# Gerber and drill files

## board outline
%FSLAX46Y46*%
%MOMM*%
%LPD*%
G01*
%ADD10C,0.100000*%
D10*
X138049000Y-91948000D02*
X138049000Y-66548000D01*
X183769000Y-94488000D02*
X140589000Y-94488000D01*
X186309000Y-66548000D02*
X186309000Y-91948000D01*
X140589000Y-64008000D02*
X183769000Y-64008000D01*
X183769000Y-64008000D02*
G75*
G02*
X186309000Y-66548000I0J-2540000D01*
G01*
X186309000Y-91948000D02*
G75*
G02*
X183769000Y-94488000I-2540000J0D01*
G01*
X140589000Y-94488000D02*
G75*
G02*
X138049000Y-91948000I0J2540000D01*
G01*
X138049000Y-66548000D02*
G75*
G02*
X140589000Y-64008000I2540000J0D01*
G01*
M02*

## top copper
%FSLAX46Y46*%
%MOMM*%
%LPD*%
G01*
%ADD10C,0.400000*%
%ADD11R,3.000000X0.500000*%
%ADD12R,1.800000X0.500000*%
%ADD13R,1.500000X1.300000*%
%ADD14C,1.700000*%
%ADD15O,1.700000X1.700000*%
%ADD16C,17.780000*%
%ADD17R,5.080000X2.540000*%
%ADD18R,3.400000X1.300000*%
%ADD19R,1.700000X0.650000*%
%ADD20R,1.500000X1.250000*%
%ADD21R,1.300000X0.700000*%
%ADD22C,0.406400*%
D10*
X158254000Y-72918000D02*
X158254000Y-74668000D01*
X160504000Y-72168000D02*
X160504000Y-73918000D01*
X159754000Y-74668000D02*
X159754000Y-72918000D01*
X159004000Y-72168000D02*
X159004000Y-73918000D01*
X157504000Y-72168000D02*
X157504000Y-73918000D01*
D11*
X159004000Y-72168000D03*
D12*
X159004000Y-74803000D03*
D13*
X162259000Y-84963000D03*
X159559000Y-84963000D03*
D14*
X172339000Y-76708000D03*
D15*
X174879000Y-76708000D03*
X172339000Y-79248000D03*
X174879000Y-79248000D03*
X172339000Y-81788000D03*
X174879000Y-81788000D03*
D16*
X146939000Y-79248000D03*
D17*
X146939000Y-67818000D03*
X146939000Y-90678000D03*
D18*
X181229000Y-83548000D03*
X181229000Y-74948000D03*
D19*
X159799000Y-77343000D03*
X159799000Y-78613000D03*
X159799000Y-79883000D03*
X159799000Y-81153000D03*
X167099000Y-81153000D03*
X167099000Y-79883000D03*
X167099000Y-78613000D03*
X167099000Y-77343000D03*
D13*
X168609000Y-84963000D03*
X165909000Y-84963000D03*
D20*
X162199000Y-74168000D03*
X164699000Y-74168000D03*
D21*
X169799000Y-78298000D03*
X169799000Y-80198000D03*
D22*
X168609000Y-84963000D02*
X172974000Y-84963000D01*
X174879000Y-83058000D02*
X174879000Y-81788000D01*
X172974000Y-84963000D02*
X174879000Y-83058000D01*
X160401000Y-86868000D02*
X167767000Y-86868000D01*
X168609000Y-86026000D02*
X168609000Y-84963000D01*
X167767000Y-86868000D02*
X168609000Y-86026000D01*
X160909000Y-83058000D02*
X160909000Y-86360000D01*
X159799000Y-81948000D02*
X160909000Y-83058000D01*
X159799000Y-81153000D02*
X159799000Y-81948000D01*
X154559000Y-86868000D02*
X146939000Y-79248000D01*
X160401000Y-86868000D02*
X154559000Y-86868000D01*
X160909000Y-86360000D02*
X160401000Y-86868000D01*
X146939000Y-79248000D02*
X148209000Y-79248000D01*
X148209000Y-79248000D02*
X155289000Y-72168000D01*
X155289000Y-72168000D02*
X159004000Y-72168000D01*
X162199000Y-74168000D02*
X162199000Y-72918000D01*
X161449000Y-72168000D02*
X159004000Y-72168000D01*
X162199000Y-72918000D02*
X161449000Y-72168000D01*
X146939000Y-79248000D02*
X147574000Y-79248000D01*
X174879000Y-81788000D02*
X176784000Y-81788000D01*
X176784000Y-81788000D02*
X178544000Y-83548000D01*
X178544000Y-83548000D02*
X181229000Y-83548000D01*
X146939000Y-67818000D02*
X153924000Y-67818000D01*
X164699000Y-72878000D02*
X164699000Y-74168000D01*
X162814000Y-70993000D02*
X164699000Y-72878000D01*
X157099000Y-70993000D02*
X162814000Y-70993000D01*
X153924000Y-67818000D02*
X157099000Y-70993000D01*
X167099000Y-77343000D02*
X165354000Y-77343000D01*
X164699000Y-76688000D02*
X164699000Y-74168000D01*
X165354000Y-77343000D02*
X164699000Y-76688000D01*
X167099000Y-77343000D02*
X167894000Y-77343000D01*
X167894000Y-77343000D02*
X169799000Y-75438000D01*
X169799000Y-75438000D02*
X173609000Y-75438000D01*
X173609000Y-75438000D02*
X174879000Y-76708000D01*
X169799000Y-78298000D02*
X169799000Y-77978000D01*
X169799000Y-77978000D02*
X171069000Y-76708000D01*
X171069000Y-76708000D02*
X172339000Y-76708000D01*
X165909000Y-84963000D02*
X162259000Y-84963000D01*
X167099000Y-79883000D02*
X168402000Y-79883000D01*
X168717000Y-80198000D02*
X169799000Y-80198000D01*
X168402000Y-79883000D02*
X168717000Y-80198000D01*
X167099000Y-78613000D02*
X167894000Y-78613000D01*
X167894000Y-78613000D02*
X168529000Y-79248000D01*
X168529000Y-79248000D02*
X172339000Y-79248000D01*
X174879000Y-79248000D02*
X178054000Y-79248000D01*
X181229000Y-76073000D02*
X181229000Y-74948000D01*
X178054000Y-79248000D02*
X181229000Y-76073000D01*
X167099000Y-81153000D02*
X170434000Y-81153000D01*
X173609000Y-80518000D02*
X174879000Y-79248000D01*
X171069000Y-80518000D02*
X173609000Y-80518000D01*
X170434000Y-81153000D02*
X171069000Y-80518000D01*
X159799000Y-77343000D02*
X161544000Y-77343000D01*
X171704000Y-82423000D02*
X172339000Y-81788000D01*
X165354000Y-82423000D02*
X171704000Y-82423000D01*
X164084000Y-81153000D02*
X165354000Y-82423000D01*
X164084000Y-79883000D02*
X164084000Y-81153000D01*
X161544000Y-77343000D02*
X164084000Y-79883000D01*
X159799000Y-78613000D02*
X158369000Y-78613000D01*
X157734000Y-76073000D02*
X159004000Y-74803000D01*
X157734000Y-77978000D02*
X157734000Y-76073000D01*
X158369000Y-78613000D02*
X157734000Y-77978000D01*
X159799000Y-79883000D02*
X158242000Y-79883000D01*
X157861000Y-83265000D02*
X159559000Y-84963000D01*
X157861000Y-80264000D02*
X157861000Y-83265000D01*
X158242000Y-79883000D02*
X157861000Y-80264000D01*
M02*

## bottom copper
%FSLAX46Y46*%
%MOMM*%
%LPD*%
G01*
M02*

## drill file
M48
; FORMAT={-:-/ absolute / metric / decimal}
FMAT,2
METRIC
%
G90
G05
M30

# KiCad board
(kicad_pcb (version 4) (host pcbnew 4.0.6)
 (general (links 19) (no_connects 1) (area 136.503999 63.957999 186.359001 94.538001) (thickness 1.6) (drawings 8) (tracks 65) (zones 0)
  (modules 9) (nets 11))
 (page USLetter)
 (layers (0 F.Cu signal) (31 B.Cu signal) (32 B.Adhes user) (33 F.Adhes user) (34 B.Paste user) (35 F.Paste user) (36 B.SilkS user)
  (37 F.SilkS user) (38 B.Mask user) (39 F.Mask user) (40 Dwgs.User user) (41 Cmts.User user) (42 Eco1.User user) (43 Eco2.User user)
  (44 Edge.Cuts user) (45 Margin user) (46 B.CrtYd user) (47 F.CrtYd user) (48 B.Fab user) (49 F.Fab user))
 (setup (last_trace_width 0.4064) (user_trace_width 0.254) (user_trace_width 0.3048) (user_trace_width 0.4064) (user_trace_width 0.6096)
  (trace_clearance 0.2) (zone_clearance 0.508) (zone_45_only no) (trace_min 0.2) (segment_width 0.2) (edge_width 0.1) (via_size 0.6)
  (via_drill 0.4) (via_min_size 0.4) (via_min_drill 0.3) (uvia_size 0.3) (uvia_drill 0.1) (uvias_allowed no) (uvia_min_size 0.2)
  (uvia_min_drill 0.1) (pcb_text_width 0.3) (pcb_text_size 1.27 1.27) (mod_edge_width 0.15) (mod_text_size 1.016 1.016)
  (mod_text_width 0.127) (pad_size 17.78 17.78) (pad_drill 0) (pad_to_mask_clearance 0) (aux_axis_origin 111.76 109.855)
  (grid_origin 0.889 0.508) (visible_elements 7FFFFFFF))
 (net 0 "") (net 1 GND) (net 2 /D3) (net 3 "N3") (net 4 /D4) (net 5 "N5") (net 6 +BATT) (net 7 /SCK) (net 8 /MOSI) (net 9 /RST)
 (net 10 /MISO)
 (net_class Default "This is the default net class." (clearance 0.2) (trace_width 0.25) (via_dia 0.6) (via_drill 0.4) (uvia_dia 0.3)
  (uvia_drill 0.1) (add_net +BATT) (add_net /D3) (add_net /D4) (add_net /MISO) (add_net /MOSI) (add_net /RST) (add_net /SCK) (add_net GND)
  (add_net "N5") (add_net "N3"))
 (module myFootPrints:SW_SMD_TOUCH (layer F.Cu) (at 159.004 74.168)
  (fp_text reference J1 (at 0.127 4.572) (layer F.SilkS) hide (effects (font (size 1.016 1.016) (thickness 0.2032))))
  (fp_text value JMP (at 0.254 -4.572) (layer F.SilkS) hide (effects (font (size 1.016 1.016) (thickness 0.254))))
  (fp_line (start -0.75 -1.25) (end -0.75 0.5) (layer F.Cu) (width 0.4))
  (fp_line (start 1.5 -2) (end 1.5 -0.25) (layer F.Cu) (width 0.4))
  (fp_line (start 0.75 0.5) (end 0.75 -1.25) (layer F.Cu) (width 0.4))
  (fp_line (start 0 -2) (end 0 -0.25) (layer F.Cu) (width 0.4))
  (fp_line (start -1.5 -2) (end -1.5 -0.25) (layer F.Cu) (width 0.4))
  (pad 1 smd rect (at 0 -2) (size 3 0.5) (layers F.Cu F.Paste F.Mask) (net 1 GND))
  (pad 2 smd rect (at 0 0.635) (size 1.8 0.5) (layers F.Cu F.Paste F.Mask) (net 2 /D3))
  (pad 3 smd circle (at 0 -0.75) (size 3.5 3.5) (layers F.Paste F.Mask)))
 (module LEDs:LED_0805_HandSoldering (layer F.Cu) (at 160.909 84.963 180)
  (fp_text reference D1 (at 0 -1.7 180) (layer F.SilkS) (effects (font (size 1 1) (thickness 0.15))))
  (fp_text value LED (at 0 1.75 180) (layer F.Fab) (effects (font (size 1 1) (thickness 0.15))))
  (pad 1 smd rect (at -1.35 0 180) (size 1.5 1.3) (layers F.Cu F.Paste F.Mask) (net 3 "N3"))
  (pad 2 smd rect (at 1.35 0 180) (size 1.5 1.3) (layers F.Cu F.Paste F.Mask) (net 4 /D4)))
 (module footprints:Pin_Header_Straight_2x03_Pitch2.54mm (layer F.Cu) (at 172.339 76.708)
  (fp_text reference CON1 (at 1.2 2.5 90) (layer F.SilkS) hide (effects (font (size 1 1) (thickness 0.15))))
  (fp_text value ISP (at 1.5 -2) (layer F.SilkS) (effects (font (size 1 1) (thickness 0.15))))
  (pad 1 smd circle (at 0 0) (size 1.7 1.7) (layers F.Cu F.Paste F.Mask) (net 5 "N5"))
  (pad 2 smd oval (at 2.54 0) (size 1.7 1.7) (layers F.Cu F.Paste F.Mask) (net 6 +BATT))
  (pad 3 smd oval (at 0 2.54) (size 1.7 1.7) (layers F.Cu F.Paste F.Mask) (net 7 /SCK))
  (pad 4 smd oval (at 2.54 2.54) (size 1.7 1.7) (layers F.Cu F.Paste F.Mask) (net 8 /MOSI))
  (pad 5 smd oval (at 0 5.08) (size 1.7 1.7) (layers F.Cu F.Paste F.Mask) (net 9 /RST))
  (pad 6 smd oval (at 2.54 5.08) (size 1.7 1.7) (layers F.Cu F.Paste F.Mask) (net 1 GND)))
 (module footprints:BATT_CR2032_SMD (layer F.Cu) (at 146.939 79.248 270)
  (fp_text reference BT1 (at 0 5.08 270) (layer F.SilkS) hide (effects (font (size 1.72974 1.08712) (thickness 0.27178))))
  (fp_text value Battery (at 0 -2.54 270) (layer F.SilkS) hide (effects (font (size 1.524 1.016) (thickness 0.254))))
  (pad 2 smd circle (at 0 0 270) (size 17.78 17.78) (layers F.Cu F.Paste F.Mask) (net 1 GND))
  (pad 1 smd rect (at -11.43 0 270) (size 2.54 5.08) (layers F.Cu F.Paste F.Mask) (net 6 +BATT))
  (pad 1 smd rect (at 11.43 0 270) (size 2.54 5.08) (layers F.Cu F.Paste F.Mask) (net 6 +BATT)))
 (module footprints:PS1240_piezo (layer F.Cu) (at 181.229 79.248 90)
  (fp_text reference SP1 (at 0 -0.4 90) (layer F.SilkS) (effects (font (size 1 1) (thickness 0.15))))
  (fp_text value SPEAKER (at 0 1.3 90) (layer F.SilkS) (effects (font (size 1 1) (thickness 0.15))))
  (pad 1 smd rect (at -4.3 0 90) (size 1.3 3.4) (layers F.Cu F.Paste F.Mask) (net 1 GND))
  (pad 2 smd rect (at 4.3 0 90) (size 1.3 3.4) (layers F.Cu F.Paste F.Mask) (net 8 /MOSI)))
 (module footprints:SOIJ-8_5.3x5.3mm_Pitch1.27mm (layer F.Cu) (at 163.449 79.248)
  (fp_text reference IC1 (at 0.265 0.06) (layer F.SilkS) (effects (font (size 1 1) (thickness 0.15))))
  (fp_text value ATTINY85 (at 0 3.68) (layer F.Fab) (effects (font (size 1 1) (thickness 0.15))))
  (pad 1 smd rect (at -3.65 -1.905) (size 1.7 0.65) (layers F.Cu F.Paste F.Mask) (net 9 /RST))
  (pad 2 smd rect (at -3.65 -0.635) (size 1.7 0.65) (layers F.Cu F.Paste F.Mask) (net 2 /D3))
  (pad 3 smd rect (at -3.65 0.635) (size 1.7 0.65) (layers F.Cu F.Paste F.Mask) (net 4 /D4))
  (pad 4 smd rect (at -3.65 1.905) (size 1.7 0.65) (layers F.Cu F.Paste F.Mask) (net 1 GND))
  (pad 5 smd rect (at 3.65 1.905) (size 1.7 0.65) (layers F.Cu F.Paste F.Mask) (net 8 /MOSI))
  (pad 6 smd rect (at 3.65 0.635) (size 1.7 0.65) (layers F.Cu F.Paste F.Mask) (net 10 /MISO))
  (pad 7 smd rect (at 3.65 -0.635) (size 1.7 0.65) (layers F.Cu F.Paste F.Mask) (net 7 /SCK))
  (pad 8 smd rect (at 3.65 -1.905) (size 1.7 0.65) (layers F.Cu F.Paste F.Mask) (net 6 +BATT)))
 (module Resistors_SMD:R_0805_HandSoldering (layer F.Cu) (at 167.259 84.963 180)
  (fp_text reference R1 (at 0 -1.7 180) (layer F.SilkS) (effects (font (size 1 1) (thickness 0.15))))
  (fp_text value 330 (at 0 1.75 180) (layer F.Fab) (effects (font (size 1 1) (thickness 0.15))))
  (pad 1 smd rect (at -1.35 0 180) (size 1.5 1.3) (layers F.Cu F.Paste F.Mask) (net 1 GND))
  (pad 2 smd rect (at 1.35 0 180) (size 1.5 1.3) (layers F.Cu F.Paste F.Mask) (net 3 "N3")))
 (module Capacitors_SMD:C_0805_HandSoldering (layer F.Cu) (at 163.449 74.168)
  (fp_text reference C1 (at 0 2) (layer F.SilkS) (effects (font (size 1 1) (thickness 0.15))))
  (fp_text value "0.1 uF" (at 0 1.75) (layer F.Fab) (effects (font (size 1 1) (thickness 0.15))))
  (pad 1 smd rect (at -1.25 0) (size 1.5 1.25) (layers F.Cu F.Paste F.Mask) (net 1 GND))
  (pad 2 smd rect (at 1.25 0) (size 1.5 1.25) (layers F.Cu F.Paste F.Mask) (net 6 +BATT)))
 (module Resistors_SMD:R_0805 (layer F.Cu) (at 169.799 79.248 270)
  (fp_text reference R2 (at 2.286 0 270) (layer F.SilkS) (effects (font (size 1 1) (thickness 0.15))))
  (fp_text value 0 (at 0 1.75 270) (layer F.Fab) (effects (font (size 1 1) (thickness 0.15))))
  (pad 1 smd rect (at -0.95 0 270) (size 0.7 1.3) (layers F.Cu F.Paste F.Mask) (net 5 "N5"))
  (pad 2 smd rect (at 0.95 0 270) (size 0.7 1.3) (layers F.Cu F.Paste F.Mask) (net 10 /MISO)))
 (gr_line (start 138.049 91.948) (end 138.049 66.548) (angle 90) (layer Edge.Cuts) (width 0.1))
 (gr_line (start 183.769 94.488) (end 140.589 94.488) (angle 90) (layer Edge.Cuts) (width 0.1))
 (gr_line (start 186.309 66.548) (end 186.309 91.948) (angle 90) (layer Edge.Cuts) (width 0.1))
 (gr_line (start 140.589 64.008) (end 183.769 64.008) (angle 90) (layer Edge.Cuts) (width 0.1))
 (gr_arc (start 183.769 66.548) (end 183.769 64.008) (angle 90) (layer Edge.Cuts) (width 0.1))
 (gr_arc (start 183.769 91.948) (end 186.309 91.948) (angle 90) (layer Edge.Cuts) (width 0.1))
 (gr_arc (start 140.589 91.948) (end 140.589 94.488) (angle 90) (layer Edge.Cuts) (width 0.1))
 (gr_arc (start 140.589 66.548) (end 138.049 66.548) (angle 90) (layer Edge.Cuts) (width 0.1))
 (segment (start 168.609 84.963) (end 172.974 84.963) (width 0.4064) (layer F.Cu) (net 1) (status 400000))
 (segment (start 174.879 83.058) (end 174.879 81.788) (width 0.4064) (layer F.Cu) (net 1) (status 800000))
 (segment (start 172.974 84.963) (end 174.879 83.058) (width 0.4064) (layer F.Cu) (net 1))
 (segment (start 160.401 86.868) (end 167.767 86.868) (width 0.4064) (layer F.Cu) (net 1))
 (segment (start 168.609 86.026) (end 168.609 84.963) (width 0.4064) (layer F.Cu) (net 1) (status 800000))
 (segment (start 167.767 86.868) (end 168.609 86.026) (width 0.4064) (layer F.Cu) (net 1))
 (segment (start 160.909 83.058) (end 160.909 86.36) (width 0.4064) (layer F.Cu) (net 1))
 (segment (start 159.799 81.948) (end 160.909 83.058) (width 0.4064) (layer F.Cu) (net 1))
 (segment (start 159.799 81.153) (end 159.799 81.948) (width 0.4064) (layer F.Cu) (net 1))
 (segment (start 154.559 86.868) (end 146.939 79.248) (width 0.4064) (layer F.Cu) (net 1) (status 800000))
 (segment (start 160.401 86.868) (end 154.559 86.868) (width 0.4064) (layer F.Cu) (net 1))
 (segment (start 160.909 86.36) (end 160.401 86.868) (width 0.4064) (layer F.Cu) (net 1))
 (segment (start 146.939 79.248) (end 148.209 79.248) (width 0.4064) (layer F.Cu) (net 1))
 (segment (start 148.209 79.248) (end 155.289 72.168) (width 0.4064) (layer F.Cu) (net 1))
 (segment (start 155.289 72.168) (end 159.004 72.168) (width 0.4064) (layer F.Cu) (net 1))
 (segment (start 162.199 74.168) (end 162.199 72.918) (width 0.4064) (layer F.Cu) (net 1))
 (segment (start 161.449 72.168) (end 159.004 72.168) (width 0.4064) (layer F.Cu) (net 1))
 (segment (start 162.199 72.918) (end 161.449 72.168) (width 0.4064) (layer F.Cu) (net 1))
 (segment (start 146.939 79.248) (end 147.574 79.248) (width 0.4064) (layer F.Cu) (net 1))
 (segment (start 174.879 81.788) (end 176.784 81.788) (width 0.4064) (layer F.Cu) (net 1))
 (segment (start 176.784 81.788) (end 178.544 83.548) (width 0.4064) (layer F.Cu) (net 1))
 (segment (start 178.544 83.548) (end 181.229 83.548) (width 0.4064) (layer F.Cu) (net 1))
 (segment (start 146.939 67.818) (end 153.924 67.818) (width 0.4064) (layer F.Cu) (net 6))
 (segment (start 164.699 72.878) (end 164.699 74.168) (width 0.4064) (layer F.Cu) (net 6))
 (segment (start 162.814 70.993) (end 164.699 72.878) (width 0.4064) (layer F.Cu) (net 6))
 (segment (start 157.099 70.993) (end 162.814 70.993) (width 0.4064) (layer F.Cu) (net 6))
 (segment (start 153.924 67.818) (end 157.099 70.993) (width 0.4064) (layer F.Cu) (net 6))
 (segment (start 167.099 77.343) (end 165.354 77.343) (width 0.4064) (layer F.Cu) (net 6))
 (segment (start 164.699 76.688) (end 164.699 74.168) (width 0.4064) (layer F.Cu) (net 6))
 (segment (start 165.354 77.343) (end 164.699 76.688) (width 0.4064) (layer F.Cu) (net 6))
 (segment (start 167.099 77.343) (end 167.894 77.343) (width 0.4064) (layer F.Cu) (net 6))
 (segment (start 167.894 77.343) (end 169.799 75.438) (width 0.4064) (layer F.Cu) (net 6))
 (segment (start 169.799 75.438) (end 173.609 75.438) (width 0.4064) (layer F.Cu) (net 6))
 (segment (start 173.609 75.438) (end 174.879 76.708) (width 0.4064) (layer F.Cu) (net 6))
 (segment (start 169.799 78.298) (end 169.799 77.978) (width 0.4064) (layer F.Cu) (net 5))
 (segment (start 169.799 77.978) (end 171.069 76.708) (width 0.4064) (layer F.Cu) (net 5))
 (segment (start 171.069 76.708) (end 172.339 76.708) (width 0.4064) (layer F.Cu) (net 5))
 (segment (start 165.909 84.963) (end 162.259 84.963) (width 0.4064) (layer F.Cu) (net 3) (status 20))
 (segment (start 167.099 79.883) (end 168.402 79.883) (width 0.4064) (layer F.Cu) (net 10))
 (segment (start 168.717 80.198) (end 169.799 80.198) (width 0.4064) (layer F.Cu) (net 10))
 (segment (start 168.402 79.883) (end 168.717 80.198) (width 0.4064) (layer F.Cu) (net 10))
 (segment (start 167.099 78.613) (end 167.894 78.613) (width 0.4064) (layer F.Cu) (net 7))
 (segment (start 167.894 78.613) (end 168.529 79.248) (width 0.4064) (layer F.Cu) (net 7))
 (segment (start 168.529 79.248) (end 172.339 79.248) (width 0.4064) (layer F.Cu) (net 7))
 (segment (start 174.879 79.248) (end 178.054 79.248) (width 0.4064) (layer F.Cu) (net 8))
 (segment (start 181.229 76.073) (end 181.229 74.948) (width 0.4064) (layer F.Cu) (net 8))
 (segment (start 178.054 79.248) (end 181.229 76.073) (width 0.4064) (layer F.Cu) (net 8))
 (segment (start 167.099 81.153) (end 170.434 81.153) (width 0.4064) (layer F.Cu) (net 8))
 (segment (start 173.609 80.518) (end 174.879 79.248) (width 0.4064) (layer F.Cu) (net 8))
 (segment (start 171.069 80.518) (end 173.609 80.518) (width 0.4064) (layer F.Cu) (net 8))
 (segment (start 170.434 81.153) (end 171.069 80.518) (width 0.4064) (layer F.Cu) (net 8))
 (segment (start 159.799 77.343) (end 161.544 77.343) (width 0.4064) (layer F.Cu) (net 9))
 (segment (start 171.704 82.423) (end 172.339 81.788) (width 0.4064) (layer F.Cu) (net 9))
 (segment (start 165.354 82.423) (end 171.704 82.423) (width 0.4064) (layer F.Cu) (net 9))
 (segment (start 164.084 81.153) (end 165.354 82.423) (width 0.4064) (layer F.Cu) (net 9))
 (segment (start 164.084 79.883) (end 164.084 81.153) (width 0.4064) (layer F.Cu) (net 9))
 (segment (start 161.544 77.343) (end 164.084 79.883) (width 0.4064) (layer F.Cu) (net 9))
 (segment (start 159.799 78.613) (end 158.369 78.613) (width 0.4064) (layer F.Cu) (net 2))
 (segment (start 157.734 76.073) (end 159.004 74.803) (width 0.4064) (layer F.Cu) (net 2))
 (segment (start 157.734 77.978) (end 157.734 76.073) (width 0.4064) (layer F.Cu) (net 2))
 (segment (start 158.369 78.613) (end 157.734 77.978) (width 0.4064) (layer F.Cu) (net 2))
 (segment (start 159.799 79.883) (end 158.242 79.883) (width 0.4064) (layer F.Cu) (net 4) (status 400000))
 (segment (start 157.861 83.265) (end 159.559 84.963) (width 0.4064) (layer F.Cu) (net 4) (status 800000))
 (segment (start 157.861 80.264) (end 157.861 83.265) (width 0.4064) (layer F.Cu) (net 4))
 (segment (start 158.242 79.883) (end 157.861 80.264) (width 0.4064) (layer F.Cu) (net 4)))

